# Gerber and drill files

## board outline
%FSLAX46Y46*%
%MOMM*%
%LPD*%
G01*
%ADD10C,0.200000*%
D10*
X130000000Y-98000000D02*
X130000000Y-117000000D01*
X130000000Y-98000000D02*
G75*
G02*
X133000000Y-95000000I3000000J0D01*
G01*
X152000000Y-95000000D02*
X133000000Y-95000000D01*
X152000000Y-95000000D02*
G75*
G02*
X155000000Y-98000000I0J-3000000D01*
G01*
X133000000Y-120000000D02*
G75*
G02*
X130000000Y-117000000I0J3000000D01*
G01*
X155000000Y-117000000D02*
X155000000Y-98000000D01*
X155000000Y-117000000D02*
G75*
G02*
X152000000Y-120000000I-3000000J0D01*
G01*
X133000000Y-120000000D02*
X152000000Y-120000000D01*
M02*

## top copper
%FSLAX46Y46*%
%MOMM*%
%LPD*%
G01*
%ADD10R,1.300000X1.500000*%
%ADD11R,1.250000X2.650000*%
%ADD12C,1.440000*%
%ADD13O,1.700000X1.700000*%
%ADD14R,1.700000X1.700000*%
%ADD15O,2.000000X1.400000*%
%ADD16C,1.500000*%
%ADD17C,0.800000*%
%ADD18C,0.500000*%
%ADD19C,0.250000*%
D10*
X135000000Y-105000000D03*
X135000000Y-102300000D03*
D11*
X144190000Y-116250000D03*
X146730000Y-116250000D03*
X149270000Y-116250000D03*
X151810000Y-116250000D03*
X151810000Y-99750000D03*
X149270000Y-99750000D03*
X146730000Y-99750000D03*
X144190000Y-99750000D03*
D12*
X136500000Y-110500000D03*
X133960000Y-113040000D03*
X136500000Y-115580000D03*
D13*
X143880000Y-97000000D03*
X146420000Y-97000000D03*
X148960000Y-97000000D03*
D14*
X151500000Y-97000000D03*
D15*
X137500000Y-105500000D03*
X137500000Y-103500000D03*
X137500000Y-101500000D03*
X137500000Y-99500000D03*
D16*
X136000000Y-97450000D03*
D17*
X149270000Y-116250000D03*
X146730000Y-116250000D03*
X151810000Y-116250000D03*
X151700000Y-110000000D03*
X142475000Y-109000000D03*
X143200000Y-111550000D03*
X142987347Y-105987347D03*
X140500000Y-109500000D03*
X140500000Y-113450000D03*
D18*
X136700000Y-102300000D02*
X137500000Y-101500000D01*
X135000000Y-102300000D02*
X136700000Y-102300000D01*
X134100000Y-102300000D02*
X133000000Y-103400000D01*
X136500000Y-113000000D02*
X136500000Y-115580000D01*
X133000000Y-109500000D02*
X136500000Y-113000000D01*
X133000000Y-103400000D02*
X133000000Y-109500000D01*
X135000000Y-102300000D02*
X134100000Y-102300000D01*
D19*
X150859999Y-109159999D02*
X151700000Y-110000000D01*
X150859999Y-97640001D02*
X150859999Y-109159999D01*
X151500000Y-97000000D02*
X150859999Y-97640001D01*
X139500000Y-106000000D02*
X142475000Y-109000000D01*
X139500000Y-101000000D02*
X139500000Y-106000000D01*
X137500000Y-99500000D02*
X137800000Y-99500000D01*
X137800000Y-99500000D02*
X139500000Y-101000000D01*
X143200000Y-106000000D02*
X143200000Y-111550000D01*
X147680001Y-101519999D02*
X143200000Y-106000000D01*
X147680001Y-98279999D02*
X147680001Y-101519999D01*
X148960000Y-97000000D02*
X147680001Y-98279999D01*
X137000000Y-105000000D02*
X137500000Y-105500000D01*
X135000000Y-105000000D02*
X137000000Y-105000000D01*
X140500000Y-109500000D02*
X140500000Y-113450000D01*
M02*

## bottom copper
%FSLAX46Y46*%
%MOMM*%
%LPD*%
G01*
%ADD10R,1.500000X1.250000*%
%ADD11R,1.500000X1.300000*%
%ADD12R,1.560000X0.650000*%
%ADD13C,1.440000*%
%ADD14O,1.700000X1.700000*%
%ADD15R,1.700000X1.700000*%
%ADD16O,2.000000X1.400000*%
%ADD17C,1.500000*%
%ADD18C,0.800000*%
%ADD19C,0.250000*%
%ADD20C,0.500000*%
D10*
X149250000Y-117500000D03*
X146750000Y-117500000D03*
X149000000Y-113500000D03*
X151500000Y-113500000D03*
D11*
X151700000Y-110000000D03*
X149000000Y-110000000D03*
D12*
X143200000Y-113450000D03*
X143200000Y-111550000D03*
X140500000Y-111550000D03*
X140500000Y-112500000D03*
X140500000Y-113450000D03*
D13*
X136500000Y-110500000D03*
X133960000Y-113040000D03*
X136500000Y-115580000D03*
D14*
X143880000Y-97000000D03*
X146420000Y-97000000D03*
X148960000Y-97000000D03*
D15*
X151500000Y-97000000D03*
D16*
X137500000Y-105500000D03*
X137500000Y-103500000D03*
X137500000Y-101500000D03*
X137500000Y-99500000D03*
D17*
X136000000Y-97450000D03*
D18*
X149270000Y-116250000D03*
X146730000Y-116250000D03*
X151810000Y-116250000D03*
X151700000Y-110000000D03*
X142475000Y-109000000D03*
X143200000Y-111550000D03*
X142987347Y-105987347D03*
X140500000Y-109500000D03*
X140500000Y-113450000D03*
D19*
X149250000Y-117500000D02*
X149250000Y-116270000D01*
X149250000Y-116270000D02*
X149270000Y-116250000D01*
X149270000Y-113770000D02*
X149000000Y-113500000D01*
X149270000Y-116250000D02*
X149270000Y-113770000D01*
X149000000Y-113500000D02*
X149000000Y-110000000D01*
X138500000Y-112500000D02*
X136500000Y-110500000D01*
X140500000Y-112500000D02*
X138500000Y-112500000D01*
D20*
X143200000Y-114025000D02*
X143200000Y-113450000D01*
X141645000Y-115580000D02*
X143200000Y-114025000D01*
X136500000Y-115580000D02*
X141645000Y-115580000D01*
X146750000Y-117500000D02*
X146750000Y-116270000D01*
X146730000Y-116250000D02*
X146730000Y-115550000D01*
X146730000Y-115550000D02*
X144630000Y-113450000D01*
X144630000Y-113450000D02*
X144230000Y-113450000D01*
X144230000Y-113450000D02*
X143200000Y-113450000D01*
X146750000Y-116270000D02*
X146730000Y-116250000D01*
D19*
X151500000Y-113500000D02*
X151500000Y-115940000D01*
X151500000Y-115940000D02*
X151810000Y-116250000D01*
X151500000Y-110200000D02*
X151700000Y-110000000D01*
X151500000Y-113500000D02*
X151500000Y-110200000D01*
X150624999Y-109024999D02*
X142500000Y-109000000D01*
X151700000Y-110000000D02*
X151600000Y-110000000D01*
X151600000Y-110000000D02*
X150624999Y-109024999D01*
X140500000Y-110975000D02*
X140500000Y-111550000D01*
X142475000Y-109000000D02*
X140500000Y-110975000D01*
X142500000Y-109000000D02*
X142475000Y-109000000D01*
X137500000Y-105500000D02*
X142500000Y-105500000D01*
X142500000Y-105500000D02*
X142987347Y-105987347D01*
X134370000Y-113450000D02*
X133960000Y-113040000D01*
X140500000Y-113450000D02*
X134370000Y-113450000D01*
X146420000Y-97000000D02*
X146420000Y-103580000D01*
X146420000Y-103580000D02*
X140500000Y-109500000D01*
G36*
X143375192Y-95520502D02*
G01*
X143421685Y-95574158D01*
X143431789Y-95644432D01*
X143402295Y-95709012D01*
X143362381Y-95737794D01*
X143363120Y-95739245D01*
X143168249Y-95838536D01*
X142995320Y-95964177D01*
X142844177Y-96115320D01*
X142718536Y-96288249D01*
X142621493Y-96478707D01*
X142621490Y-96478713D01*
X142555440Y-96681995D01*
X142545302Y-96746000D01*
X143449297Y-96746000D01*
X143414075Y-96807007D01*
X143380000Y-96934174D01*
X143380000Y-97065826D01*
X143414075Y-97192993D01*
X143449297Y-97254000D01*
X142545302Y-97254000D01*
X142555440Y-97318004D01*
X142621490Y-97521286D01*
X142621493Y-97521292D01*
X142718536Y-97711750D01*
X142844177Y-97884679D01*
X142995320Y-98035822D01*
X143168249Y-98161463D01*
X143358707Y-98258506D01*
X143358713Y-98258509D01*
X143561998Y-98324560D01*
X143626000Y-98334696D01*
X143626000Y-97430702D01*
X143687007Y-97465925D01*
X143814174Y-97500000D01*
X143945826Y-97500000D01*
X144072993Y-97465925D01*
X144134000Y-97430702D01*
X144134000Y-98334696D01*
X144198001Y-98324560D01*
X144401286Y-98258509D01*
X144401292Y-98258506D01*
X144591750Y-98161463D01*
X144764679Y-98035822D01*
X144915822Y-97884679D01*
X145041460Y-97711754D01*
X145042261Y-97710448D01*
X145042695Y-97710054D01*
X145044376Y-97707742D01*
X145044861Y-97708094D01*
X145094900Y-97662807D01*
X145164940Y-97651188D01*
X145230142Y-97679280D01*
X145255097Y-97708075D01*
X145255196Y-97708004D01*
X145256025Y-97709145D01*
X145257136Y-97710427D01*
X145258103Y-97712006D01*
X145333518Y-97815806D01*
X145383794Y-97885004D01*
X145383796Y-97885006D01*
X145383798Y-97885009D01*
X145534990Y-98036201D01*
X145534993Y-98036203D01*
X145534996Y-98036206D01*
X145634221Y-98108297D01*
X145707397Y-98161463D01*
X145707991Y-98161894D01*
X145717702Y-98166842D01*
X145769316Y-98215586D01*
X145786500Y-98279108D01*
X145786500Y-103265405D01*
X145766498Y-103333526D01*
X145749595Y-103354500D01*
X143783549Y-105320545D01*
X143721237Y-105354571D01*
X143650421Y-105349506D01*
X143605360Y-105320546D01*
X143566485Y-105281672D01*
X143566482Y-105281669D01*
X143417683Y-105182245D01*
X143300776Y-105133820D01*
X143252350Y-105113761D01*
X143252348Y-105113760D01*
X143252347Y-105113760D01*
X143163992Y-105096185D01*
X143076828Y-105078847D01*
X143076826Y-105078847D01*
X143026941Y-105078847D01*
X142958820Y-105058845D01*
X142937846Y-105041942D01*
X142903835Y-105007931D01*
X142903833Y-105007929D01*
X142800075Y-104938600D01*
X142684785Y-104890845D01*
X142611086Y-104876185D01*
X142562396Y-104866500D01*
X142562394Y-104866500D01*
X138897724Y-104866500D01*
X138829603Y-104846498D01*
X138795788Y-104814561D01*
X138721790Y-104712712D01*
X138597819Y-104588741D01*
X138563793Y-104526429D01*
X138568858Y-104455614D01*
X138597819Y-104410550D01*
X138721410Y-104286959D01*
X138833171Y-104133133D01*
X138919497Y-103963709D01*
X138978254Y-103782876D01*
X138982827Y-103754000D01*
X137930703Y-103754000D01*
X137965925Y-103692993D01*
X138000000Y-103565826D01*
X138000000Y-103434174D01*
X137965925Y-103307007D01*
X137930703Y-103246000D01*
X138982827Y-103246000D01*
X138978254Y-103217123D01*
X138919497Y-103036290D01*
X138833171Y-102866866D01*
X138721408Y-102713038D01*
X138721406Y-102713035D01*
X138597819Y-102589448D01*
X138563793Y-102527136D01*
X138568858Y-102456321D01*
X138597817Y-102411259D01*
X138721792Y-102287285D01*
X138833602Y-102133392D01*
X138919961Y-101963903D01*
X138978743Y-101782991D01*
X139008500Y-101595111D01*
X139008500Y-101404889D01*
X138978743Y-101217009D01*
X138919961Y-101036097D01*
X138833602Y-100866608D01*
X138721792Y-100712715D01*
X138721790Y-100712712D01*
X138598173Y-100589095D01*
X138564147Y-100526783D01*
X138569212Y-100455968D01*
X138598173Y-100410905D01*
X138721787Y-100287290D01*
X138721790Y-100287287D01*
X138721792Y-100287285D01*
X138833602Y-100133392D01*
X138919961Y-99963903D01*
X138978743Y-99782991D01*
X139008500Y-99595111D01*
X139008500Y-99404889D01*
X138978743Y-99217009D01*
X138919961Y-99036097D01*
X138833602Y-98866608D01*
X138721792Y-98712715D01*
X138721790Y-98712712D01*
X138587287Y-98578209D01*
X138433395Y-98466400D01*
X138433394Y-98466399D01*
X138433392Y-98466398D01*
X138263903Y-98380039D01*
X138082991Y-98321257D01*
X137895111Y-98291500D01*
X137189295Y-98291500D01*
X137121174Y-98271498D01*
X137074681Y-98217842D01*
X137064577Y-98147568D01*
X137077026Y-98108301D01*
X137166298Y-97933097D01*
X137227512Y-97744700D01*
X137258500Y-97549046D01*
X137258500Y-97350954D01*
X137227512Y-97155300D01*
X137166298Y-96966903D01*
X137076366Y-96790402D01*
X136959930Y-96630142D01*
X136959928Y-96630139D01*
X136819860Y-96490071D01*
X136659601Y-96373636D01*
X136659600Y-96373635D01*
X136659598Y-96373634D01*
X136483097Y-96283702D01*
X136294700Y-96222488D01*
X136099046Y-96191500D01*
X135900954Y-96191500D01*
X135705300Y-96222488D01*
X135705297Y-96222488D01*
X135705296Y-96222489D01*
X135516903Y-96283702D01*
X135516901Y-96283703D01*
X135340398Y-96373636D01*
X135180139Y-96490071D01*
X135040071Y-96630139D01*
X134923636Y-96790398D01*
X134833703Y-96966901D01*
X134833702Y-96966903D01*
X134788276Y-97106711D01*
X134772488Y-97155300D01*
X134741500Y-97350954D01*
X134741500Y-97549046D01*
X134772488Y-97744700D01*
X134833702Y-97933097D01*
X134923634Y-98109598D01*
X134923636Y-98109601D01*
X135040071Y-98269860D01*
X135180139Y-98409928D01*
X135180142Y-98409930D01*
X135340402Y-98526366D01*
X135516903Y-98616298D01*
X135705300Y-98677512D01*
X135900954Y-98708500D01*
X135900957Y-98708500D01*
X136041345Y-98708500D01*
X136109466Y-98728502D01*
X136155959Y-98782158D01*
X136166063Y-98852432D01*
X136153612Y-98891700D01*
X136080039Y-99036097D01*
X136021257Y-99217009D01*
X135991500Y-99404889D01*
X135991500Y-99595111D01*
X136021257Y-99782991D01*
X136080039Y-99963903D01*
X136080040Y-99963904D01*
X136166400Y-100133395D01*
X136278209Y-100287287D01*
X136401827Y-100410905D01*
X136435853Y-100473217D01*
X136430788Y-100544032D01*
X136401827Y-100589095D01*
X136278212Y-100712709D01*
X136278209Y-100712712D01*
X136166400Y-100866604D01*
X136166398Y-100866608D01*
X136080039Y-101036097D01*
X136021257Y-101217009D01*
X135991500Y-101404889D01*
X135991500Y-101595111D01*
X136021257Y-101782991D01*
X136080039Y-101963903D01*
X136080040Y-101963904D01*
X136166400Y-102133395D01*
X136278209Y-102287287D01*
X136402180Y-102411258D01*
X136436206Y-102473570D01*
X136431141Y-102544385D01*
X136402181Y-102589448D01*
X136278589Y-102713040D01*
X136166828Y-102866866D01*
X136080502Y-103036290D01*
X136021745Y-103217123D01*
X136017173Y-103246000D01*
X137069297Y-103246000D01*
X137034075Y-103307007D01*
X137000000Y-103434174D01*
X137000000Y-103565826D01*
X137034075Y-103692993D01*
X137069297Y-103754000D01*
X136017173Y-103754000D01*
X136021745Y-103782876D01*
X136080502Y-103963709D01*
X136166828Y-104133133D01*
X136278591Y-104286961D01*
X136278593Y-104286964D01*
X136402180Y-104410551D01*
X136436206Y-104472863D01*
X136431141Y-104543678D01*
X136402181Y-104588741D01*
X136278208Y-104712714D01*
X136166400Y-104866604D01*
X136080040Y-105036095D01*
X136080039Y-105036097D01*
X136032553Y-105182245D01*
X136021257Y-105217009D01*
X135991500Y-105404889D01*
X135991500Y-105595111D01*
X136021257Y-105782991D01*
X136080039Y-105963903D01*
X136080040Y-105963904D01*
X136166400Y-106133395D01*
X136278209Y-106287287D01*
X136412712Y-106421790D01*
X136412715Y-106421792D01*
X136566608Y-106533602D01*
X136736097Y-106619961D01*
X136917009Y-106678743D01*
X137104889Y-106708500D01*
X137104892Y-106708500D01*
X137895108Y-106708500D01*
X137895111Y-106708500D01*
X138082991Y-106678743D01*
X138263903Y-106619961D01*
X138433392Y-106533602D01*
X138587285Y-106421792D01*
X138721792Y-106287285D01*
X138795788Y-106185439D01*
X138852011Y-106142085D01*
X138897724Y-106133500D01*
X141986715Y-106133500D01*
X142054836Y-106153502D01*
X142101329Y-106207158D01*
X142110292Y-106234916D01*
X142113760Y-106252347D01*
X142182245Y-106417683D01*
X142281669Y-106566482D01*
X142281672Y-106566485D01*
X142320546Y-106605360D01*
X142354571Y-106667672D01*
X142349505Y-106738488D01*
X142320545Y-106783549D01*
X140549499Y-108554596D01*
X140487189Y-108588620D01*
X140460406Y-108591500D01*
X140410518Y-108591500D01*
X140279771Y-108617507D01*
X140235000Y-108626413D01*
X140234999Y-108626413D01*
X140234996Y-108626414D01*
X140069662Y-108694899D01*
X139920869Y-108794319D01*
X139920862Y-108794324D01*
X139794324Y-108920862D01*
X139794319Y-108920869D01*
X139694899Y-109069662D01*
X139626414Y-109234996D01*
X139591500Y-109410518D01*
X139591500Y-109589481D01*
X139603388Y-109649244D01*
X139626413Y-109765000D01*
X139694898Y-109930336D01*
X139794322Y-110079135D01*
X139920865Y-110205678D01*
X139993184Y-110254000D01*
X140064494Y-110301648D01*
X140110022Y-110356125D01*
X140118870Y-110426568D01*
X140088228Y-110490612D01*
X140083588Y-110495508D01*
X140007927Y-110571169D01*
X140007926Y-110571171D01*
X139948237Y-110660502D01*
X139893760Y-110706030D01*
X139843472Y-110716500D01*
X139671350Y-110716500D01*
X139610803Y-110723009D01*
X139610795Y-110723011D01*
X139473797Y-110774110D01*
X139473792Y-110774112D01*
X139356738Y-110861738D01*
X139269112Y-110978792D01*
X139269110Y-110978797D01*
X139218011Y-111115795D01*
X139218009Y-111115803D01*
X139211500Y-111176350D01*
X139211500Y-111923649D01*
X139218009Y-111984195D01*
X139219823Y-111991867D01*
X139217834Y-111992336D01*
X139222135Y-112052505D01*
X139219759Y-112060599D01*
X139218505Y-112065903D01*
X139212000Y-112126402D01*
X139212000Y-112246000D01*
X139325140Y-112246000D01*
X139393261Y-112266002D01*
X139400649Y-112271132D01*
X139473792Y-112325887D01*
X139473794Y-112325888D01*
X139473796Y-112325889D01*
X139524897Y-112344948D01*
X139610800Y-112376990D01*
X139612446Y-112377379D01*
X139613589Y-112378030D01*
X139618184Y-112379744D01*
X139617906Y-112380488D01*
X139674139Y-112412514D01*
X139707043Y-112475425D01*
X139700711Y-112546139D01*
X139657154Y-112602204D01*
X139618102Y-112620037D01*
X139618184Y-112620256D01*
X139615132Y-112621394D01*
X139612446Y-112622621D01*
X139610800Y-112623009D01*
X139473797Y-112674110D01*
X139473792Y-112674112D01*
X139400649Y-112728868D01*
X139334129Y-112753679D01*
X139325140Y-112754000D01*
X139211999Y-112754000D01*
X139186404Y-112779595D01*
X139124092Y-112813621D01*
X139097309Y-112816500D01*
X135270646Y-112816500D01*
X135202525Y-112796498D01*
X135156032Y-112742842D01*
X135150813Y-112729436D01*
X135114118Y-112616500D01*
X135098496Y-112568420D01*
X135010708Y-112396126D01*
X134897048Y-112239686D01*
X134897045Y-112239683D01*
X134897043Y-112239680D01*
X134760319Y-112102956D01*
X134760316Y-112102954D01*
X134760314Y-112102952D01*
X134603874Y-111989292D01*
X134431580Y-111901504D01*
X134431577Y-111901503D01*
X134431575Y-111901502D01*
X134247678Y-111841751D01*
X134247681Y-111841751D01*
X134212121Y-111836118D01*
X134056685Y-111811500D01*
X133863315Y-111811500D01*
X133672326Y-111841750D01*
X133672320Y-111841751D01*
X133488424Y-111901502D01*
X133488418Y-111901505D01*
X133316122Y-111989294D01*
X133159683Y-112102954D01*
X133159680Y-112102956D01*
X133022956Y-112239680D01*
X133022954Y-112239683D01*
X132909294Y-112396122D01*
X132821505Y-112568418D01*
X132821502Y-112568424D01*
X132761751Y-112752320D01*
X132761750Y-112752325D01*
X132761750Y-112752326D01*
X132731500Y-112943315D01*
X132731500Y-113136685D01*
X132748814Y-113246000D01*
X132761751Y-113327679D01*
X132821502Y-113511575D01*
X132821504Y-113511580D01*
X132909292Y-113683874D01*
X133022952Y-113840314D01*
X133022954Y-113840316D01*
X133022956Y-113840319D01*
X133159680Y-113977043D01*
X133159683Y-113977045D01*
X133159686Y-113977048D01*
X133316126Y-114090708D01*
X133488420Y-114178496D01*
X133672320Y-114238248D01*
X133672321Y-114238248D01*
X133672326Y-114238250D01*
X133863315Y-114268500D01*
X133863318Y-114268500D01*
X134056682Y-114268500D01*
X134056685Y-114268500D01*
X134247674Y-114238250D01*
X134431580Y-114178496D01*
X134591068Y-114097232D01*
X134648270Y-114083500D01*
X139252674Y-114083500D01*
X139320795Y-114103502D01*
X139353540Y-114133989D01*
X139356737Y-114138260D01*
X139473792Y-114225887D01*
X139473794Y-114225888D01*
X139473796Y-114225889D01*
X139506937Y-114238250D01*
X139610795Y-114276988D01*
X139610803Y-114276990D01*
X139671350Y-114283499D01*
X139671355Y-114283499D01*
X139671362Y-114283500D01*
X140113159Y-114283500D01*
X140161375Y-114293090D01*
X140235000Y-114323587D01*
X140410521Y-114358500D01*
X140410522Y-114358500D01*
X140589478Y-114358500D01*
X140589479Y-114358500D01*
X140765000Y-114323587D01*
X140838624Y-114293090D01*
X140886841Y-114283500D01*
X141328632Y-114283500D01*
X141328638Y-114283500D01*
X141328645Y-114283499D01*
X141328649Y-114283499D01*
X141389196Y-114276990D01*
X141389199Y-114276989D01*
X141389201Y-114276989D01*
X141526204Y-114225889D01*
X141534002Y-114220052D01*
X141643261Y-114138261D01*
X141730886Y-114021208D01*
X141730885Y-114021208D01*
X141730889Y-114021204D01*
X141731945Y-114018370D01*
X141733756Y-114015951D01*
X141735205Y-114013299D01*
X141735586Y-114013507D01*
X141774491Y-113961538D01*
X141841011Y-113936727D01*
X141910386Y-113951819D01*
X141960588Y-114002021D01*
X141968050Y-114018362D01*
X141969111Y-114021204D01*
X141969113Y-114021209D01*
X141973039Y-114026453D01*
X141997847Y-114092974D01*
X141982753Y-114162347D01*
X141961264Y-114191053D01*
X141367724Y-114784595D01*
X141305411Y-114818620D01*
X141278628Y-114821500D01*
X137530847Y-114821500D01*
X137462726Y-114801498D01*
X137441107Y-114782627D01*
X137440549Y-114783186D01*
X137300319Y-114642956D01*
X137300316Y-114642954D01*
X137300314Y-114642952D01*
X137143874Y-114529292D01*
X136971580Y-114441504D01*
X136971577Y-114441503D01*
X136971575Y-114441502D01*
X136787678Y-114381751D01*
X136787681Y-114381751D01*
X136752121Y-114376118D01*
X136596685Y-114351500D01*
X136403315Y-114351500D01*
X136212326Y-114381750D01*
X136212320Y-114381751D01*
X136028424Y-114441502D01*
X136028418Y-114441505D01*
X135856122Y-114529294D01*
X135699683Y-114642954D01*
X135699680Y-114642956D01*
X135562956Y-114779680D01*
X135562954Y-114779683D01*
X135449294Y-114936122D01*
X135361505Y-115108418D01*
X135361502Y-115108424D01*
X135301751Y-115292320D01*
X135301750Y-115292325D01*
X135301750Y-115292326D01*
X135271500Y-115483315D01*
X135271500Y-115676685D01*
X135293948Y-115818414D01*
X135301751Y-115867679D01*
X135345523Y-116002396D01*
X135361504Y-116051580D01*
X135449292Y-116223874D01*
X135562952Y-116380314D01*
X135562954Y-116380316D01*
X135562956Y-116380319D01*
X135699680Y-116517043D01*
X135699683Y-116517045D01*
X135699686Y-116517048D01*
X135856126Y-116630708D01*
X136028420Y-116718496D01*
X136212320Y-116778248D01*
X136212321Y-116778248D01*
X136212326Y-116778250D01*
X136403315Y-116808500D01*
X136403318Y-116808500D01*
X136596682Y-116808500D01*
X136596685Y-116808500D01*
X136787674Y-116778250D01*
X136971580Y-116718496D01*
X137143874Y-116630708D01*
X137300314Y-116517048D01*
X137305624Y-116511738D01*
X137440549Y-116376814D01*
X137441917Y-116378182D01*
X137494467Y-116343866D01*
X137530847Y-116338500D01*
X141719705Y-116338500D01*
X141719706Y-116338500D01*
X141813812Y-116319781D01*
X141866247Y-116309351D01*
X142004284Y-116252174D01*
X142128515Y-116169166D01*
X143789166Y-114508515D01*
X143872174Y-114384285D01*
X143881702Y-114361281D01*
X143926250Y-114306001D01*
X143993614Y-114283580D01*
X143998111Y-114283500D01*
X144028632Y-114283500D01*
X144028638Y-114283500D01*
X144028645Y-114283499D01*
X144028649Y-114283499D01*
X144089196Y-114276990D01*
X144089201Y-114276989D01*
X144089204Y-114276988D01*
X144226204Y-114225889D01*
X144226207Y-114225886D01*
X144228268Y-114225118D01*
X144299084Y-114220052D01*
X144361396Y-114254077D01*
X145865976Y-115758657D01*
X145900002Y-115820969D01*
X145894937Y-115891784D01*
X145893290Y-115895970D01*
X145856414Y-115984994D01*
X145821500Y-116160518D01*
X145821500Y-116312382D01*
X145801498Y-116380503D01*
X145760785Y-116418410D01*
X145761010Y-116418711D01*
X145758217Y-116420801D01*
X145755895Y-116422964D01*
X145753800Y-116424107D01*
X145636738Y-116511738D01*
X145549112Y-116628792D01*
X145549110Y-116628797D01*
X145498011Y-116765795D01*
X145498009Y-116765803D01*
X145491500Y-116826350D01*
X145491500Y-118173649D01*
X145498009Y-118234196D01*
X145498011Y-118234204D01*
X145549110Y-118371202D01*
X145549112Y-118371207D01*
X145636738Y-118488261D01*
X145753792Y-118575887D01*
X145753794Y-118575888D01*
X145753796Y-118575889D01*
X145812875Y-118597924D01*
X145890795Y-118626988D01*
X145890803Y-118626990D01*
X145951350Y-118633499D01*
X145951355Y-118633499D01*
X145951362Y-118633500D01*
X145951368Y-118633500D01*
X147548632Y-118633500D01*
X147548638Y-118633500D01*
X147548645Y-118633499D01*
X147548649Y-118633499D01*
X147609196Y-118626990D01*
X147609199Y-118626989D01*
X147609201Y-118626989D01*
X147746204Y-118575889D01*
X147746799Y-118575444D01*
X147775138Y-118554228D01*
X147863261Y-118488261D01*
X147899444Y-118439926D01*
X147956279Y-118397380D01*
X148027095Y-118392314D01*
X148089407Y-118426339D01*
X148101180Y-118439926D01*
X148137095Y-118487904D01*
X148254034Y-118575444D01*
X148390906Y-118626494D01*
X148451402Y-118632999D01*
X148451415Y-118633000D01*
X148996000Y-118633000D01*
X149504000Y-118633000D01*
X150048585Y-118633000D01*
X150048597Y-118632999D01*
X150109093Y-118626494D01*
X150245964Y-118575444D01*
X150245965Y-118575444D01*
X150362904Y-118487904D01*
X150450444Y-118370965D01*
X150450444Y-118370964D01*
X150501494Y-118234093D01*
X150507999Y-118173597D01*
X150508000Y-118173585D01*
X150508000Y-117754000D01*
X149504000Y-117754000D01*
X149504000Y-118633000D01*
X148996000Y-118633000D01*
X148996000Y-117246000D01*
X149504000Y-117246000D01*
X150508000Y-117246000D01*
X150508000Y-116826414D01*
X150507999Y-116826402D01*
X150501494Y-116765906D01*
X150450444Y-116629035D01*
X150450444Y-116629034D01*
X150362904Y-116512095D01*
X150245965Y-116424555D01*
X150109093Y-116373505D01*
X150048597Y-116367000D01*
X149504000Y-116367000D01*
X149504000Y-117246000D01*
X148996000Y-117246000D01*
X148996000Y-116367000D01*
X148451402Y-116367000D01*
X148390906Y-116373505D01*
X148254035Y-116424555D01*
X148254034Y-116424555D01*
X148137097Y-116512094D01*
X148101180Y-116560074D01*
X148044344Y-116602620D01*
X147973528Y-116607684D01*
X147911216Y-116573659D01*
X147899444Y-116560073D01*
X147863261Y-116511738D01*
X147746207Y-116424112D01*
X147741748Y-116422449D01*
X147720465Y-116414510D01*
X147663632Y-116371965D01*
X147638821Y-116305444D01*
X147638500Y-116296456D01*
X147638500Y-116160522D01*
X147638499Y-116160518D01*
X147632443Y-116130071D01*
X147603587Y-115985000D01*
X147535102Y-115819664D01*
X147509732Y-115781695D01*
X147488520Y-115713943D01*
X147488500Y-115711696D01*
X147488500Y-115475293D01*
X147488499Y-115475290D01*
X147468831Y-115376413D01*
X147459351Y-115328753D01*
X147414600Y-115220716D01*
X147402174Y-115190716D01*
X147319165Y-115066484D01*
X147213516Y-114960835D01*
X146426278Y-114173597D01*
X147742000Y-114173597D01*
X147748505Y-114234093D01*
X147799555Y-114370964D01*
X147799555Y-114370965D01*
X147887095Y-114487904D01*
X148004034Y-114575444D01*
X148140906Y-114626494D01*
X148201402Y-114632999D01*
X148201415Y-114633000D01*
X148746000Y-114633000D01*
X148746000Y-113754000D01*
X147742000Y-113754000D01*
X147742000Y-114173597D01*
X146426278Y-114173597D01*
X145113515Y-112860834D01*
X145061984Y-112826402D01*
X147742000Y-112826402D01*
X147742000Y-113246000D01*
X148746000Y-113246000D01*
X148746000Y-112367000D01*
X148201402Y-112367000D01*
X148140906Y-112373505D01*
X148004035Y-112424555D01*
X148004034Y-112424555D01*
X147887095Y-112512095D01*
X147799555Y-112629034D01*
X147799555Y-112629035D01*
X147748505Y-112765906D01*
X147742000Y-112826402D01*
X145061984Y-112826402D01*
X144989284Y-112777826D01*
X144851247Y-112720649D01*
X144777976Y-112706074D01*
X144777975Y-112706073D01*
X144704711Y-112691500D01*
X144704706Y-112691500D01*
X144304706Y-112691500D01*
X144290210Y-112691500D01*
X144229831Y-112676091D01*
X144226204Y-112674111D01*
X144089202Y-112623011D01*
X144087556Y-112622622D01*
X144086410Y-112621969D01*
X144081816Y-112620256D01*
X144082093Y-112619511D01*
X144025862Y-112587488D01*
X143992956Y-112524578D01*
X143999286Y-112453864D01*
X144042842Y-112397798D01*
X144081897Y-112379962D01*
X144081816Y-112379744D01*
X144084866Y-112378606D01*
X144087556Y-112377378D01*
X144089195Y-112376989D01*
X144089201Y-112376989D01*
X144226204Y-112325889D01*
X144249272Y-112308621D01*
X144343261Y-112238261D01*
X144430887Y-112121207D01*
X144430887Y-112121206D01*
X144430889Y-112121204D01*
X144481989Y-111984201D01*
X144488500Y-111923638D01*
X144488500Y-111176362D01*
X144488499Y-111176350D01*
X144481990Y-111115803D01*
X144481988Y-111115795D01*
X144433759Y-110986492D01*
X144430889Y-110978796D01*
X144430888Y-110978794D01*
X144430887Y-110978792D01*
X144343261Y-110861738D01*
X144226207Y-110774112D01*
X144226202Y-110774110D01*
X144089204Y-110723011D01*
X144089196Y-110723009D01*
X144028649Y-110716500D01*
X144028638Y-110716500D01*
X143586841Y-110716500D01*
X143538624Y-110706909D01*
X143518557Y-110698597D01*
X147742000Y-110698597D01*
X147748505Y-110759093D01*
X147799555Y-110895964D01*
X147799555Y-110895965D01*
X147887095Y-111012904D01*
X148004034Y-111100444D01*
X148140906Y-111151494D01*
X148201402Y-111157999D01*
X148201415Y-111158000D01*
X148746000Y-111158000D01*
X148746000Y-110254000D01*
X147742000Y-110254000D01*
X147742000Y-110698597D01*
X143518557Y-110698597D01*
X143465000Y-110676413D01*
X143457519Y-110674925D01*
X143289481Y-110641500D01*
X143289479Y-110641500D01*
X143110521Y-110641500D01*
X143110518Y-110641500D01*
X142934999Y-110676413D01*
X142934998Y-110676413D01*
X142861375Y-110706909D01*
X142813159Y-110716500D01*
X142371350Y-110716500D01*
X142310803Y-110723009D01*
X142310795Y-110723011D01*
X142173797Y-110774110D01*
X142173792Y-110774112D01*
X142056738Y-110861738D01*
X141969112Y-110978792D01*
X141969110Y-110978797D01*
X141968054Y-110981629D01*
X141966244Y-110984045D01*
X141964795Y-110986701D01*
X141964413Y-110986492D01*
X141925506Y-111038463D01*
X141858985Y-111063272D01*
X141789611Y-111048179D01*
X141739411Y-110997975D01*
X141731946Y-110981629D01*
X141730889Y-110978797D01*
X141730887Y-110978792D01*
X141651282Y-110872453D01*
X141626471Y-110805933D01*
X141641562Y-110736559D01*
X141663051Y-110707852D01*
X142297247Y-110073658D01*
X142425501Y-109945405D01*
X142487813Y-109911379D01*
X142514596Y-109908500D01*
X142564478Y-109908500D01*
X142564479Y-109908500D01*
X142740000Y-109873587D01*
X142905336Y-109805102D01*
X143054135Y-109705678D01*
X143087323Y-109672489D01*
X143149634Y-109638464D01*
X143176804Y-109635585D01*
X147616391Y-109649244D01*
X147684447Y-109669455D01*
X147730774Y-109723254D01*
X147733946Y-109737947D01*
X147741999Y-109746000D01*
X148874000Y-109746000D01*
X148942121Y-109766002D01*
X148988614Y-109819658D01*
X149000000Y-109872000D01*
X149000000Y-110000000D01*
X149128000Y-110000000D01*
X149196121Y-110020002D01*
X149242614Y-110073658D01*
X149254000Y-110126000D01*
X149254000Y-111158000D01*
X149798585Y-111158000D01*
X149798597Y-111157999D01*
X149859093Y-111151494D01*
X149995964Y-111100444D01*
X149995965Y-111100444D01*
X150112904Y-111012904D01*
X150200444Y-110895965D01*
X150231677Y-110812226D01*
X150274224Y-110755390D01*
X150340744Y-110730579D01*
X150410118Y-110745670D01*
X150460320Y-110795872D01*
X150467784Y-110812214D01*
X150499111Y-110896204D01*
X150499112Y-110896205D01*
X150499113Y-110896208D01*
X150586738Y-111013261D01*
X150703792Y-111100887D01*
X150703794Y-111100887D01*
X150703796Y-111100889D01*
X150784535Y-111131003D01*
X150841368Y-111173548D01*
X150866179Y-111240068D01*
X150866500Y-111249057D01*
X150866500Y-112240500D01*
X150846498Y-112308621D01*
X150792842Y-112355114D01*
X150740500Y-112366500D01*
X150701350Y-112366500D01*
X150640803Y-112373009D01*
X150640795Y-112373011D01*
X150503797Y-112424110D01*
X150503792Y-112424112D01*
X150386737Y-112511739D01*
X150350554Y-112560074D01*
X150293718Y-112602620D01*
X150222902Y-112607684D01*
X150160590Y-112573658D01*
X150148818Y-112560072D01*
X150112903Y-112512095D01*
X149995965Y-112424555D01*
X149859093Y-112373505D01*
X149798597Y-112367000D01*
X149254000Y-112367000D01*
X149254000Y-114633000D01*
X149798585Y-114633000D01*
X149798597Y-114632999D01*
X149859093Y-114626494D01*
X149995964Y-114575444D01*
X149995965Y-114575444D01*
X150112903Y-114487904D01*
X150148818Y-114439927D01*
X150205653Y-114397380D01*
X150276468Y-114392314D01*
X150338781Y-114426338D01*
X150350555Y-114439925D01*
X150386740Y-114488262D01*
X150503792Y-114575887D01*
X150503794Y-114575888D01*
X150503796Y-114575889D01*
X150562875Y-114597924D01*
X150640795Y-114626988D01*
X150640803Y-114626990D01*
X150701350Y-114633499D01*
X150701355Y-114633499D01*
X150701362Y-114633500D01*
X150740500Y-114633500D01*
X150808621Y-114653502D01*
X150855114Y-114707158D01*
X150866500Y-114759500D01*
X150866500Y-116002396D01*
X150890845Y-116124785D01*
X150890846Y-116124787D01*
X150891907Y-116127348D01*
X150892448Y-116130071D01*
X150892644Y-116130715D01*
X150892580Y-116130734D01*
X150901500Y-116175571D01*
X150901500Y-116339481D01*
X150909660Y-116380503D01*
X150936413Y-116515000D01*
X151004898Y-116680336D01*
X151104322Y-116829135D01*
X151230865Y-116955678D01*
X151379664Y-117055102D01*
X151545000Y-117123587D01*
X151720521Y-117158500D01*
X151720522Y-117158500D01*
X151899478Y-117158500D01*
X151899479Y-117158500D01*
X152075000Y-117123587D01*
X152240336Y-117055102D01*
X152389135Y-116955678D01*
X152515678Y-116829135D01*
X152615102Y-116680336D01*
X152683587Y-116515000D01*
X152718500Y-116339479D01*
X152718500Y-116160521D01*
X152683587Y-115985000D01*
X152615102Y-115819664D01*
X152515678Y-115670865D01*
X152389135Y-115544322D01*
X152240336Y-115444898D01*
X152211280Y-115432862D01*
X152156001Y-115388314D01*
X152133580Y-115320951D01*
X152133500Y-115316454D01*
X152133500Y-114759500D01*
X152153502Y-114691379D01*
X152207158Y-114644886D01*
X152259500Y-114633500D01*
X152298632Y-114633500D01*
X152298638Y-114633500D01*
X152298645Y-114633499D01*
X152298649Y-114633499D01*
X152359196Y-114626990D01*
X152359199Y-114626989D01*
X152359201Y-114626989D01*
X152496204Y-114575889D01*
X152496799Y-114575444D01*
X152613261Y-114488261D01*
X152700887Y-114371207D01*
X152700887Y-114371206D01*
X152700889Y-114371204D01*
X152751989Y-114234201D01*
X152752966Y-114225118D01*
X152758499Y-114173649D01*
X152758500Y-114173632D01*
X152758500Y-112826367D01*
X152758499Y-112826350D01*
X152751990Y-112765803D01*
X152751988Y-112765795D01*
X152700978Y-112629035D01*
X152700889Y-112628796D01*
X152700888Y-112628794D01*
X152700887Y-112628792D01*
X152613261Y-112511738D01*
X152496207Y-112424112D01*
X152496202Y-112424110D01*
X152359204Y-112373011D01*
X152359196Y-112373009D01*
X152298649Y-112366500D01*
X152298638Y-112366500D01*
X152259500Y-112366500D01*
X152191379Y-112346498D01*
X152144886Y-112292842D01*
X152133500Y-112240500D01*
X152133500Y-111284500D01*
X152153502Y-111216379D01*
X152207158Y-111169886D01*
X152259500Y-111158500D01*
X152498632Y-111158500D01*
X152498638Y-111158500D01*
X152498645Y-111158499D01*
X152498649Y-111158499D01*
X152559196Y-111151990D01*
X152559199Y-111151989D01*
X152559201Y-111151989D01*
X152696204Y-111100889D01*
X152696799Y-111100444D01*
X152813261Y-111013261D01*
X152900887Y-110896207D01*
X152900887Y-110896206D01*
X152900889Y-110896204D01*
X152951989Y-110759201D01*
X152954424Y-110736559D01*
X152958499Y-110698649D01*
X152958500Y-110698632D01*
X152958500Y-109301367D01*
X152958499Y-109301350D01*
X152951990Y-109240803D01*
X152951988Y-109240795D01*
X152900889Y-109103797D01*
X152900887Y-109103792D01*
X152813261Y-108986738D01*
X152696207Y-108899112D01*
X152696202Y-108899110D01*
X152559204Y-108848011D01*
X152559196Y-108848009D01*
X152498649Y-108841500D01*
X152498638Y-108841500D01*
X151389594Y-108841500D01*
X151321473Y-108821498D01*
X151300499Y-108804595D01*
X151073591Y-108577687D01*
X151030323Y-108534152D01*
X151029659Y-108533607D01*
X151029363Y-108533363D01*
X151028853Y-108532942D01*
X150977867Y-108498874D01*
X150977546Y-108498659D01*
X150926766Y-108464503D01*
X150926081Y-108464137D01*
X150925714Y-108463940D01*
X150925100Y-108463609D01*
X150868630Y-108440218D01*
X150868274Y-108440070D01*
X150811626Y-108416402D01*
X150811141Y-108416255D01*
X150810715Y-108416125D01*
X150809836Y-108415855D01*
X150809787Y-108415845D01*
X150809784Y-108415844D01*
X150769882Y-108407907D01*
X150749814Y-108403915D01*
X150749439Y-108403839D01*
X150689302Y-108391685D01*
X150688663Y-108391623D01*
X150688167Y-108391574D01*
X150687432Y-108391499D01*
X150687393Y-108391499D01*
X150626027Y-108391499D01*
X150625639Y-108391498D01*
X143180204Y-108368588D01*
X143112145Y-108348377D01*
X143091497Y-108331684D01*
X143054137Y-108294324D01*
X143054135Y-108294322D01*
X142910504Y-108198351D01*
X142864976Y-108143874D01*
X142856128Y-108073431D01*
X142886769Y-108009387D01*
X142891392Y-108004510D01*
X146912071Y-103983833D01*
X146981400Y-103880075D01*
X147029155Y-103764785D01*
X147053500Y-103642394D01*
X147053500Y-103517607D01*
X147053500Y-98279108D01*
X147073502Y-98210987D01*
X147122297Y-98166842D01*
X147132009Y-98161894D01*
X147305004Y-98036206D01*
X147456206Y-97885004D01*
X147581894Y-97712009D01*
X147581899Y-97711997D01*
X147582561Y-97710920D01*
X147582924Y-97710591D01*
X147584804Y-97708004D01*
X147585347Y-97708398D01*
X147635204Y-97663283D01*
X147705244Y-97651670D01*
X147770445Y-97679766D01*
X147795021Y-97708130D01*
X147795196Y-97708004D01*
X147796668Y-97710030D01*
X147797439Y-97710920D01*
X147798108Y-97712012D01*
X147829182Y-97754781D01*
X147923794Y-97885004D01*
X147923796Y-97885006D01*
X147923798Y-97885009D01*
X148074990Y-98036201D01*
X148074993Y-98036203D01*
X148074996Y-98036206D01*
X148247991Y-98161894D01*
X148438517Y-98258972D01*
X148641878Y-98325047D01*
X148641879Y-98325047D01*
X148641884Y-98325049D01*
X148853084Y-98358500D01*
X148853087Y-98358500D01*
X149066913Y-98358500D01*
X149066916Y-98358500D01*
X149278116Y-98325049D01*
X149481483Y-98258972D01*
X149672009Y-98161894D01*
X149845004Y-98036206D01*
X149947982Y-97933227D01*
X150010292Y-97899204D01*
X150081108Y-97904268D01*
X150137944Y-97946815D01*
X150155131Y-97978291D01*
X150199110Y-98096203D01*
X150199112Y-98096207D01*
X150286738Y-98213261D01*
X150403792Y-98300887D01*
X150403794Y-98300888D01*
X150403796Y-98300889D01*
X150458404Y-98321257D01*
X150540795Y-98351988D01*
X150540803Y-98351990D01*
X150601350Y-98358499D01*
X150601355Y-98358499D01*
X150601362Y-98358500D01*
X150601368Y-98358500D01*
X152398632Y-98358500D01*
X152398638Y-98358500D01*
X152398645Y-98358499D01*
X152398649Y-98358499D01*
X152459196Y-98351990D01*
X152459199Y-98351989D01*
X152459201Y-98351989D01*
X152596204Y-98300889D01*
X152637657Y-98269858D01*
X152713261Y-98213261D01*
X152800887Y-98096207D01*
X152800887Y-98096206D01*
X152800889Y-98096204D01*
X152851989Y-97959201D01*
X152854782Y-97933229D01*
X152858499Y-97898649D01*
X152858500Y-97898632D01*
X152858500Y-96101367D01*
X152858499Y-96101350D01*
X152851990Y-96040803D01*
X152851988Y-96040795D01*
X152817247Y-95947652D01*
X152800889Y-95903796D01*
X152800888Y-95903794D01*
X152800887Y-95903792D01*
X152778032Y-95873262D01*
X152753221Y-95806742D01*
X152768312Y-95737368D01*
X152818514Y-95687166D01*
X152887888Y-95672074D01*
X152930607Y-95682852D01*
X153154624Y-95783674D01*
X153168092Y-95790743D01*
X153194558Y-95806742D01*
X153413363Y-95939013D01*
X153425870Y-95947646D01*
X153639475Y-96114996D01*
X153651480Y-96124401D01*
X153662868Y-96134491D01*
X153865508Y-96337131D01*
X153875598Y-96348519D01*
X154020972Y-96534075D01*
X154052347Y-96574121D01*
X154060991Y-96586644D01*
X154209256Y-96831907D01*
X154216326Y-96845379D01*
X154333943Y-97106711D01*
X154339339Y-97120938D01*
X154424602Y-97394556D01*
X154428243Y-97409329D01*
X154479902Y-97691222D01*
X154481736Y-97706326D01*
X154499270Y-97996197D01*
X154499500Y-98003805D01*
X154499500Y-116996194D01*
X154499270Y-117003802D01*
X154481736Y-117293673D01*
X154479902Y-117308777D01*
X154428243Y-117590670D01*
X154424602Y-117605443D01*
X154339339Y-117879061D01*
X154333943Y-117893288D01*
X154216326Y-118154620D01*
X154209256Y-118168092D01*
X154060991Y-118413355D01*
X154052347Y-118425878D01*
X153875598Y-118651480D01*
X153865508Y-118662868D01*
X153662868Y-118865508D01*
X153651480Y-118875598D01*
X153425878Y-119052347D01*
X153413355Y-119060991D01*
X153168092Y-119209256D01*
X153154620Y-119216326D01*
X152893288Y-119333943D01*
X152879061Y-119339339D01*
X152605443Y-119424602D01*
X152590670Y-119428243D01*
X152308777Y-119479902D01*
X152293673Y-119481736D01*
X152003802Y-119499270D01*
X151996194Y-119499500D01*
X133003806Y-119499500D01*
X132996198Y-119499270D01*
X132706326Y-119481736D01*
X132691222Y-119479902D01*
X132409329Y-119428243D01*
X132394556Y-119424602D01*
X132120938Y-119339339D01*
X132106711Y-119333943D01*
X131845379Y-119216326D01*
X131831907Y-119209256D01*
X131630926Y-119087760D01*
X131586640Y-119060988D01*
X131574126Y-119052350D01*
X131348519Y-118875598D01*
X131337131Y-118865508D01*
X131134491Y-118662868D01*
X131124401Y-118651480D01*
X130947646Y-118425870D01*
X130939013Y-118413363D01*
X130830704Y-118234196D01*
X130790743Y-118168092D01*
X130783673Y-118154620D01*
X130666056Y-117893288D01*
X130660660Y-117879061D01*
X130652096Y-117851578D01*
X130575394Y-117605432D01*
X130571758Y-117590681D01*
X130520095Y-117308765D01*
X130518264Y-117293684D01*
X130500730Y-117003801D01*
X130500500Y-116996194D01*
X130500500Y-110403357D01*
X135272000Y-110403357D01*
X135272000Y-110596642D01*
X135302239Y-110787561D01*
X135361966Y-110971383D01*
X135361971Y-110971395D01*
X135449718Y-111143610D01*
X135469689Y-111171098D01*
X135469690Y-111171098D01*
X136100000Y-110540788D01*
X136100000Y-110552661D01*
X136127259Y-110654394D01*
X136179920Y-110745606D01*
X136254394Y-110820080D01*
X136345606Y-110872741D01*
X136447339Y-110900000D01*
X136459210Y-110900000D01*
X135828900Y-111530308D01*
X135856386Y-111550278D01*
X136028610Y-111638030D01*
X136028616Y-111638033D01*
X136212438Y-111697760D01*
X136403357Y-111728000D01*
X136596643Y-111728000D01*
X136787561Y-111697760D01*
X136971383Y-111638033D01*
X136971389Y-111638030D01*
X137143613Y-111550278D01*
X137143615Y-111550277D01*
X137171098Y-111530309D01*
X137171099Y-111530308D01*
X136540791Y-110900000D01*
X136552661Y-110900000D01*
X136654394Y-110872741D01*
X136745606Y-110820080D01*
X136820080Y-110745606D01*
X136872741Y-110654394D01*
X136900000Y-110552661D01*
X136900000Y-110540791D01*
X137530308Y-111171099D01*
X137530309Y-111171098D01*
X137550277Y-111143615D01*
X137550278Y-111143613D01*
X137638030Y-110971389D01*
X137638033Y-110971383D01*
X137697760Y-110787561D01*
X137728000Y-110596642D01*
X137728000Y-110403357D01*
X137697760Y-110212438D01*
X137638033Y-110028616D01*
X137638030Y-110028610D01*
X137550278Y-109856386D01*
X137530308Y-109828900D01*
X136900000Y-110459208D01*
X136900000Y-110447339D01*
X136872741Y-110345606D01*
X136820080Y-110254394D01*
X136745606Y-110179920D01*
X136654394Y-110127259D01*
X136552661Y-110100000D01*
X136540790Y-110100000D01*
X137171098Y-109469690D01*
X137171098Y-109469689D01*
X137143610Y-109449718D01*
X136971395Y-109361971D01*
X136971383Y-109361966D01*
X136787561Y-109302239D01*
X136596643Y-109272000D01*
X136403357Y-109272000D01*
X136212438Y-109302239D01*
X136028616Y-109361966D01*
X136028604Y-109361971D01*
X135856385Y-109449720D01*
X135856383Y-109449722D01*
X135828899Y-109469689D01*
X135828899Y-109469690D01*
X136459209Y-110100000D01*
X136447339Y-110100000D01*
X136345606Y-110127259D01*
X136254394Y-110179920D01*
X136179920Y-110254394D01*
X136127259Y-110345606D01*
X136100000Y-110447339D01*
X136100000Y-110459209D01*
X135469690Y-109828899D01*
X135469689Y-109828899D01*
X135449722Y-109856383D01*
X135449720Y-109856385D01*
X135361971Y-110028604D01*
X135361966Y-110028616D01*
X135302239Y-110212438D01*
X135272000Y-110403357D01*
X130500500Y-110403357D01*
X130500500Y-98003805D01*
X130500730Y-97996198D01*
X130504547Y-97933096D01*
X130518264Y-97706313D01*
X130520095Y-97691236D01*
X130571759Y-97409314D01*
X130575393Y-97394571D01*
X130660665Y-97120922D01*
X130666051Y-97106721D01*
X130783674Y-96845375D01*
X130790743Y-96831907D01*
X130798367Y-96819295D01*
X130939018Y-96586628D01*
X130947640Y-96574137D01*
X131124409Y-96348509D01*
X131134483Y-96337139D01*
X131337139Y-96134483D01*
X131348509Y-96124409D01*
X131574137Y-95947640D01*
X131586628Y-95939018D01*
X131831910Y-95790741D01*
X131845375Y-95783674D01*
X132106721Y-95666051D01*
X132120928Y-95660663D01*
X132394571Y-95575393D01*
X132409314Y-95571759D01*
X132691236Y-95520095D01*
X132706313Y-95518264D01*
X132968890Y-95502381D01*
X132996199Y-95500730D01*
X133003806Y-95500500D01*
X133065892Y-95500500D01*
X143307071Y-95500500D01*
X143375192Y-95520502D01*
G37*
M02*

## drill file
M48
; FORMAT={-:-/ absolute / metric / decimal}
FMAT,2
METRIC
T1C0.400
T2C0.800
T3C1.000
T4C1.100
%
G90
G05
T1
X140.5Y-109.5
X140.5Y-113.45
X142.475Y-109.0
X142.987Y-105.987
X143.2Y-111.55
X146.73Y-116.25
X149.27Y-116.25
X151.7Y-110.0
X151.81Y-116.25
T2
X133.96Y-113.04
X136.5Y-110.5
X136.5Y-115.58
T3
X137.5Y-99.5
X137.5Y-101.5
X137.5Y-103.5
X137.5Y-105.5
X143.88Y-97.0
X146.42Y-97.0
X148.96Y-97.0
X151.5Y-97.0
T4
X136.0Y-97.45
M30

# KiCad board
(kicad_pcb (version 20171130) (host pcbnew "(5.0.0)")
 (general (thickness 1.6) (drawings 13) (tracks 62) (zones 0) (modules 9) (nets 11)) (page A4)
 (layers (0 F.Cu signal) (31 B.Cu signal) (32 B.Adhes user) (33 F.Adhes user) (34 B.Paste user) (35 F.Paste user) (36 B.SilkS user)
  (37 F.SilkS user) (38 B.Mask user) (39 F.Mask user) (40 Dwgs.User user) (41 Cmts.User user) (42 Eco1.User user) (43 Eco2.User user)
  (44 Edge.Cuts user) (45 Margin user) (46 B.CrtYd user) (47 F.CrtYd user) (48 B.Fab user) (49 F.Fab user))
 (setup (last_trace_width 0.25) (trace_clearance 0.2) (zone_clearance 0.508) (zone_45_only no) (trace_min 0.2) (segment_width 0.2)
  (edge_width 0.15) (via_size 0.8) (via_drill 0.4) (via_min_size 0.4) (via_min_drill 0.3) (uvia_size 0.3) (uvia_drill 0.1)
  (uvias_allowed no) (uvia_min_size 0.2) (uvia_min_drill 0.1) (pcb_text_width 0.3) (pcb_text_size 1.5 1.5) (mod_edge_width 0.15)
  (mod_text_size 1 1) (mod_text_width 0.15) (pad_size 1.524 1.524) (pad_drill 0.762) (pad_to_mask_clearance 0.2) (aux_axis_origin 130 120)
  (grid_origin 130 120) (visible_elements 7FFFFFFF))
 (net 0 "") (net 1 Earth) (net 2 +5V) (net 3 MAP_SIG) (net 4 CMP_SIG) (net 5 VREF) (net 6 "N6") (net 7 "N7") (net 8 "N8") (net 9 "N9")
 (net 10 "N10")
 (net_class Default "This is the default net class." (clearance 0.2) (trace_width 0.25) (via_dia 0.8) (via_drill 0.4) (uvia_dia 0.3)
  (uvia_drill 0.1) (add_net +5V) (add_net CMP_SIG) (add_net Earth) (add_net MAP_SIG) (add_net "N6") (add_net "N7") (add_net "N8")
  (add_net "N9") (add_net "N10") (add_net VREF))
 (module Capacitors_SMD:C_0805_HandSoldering (layer B.Cu) (at 148 117.5)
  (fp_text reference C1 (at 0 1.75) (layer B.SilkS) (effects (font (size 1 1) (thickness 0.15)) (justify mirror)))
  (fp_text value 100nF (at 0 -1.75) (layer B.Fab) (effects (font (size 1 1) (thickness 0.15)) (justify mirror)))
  (pad 2 smd rect (at 1.25 0) (size 1.5 1.25) (layers B.Cu B.Paste B.Mask) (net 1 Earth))
  (pad 1 smd rect (at -1.25 0) (size 1.5 1.25) (layers B.Cu B.Paste B.Mask) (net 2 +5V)))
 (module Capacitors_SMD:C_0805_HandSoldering (layer B.Cu) (at 150.25 113.5)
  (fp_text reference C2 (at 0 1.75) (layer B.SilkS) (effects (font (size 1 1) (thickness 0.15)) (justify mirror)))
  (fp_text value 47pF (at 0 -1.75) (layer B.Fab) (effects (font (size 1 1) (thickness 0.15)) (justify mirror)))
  (pad 1 smd rect (at -1.25 0) (size 1.5 1.25) (layers B.Cu B.Paste B.Mask) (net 1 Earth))
  (pad 2 smd rect (at 1.25 0) (size 1.5 1.25) (layers B.Cu B.Paste B.Mask) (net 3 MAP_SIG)))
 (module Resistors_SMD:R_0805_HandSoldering (layer F.Cu) (at 135 103.65 270)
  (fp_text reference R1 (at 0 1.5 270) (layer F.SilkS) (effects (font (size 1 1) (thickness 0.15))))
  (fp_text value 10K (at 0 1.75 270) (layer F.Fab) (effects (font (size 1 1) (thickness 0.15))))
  (pad 2 smd rect (at 1.35 0 270) (size 1.5 1.3) (layers F.Cu F.Paste F.Mask) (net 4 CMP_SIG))
  (pad 1 smd rect (at -1.35 0 270) (size 1.5 1.3) (layers F.Cu F.Paste F.Mask) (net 2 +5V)))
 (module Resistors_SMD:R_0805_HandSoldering (layer B.Cu) (at 150.35 110 180)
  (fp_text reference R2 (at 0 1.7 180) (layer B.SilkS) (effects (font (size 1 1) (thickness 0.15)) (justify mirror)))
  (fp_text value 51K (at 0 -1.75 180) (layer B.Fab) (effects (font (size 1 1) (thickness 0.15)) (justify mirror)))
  (pad 1 smd rect (at -1.35 0 180) (size 1.5 1.3) (layers B.Cu B.Paste B.Mask) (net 3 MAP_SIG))
  (pad 2 smd rect (at 1.35 0 180) (size 1.5 1.3) (layers B.Cu B.Paste B.Mask) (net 1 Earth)))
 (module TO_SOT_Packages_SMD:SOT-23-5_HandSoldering (layer B.Cu) (at 141.85 112.5)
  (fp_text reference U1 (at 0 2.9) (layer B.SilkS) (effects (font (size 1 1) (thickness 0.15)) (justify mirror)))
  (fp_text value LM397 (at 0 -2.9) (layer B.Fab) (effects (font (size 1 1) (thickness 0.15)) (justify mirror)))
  (pad 5 smd rect (at 1.35 0.95) (size 1.56 0.65) (layers B.Cu B.Paste B.Mask) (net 2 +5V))
  (pad 4 smd rect (at 1.35 -0.95) (size 1.56 0.65) (layers B.Cu B.Paste B.Mask) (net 4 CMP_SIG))
  (pad 3 smd rect (at -1.35 -0.95) (size 1.56 0.65) (layers B.Cu B.Paste B.Mask) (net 3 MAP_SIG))
  (pad 2 smd rect (at -1.35 0) (size 1.56 0.65) (layers B.Cu B.Paste B.Mask) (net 1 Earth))
  (pad 1 smd rect (at -1.35 0.95) (size 1.56 0.65) (layers B.Cu B.Paste B.Mask) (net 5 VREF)))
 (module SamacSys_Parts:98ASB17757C (layer F.Cu) (at 148 108 90)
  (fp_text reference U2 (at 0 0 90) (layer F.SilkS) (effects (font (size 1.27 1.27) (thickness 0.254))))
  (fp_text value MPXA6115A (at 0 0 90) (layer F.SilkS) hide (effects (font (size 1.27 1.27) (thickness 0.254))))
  (pad 1 smd rect (at -8.25 -3.81 180) (size 1.25 2.65) (layers F.Cu F.Paste F.Mask) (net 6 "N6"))
  (pad 2 smd rect (at -8.25 -1.27 180) (size 1.25 2.65) (layers F.Cu F.Paste F.Mask) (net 2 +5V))
  (pad 3 smd rect (at -8.25 1.27 180) (size 1.25 2.65) (layers F.Cu F.Paste F.Mask) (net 1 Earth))
  (pad 4 smd rect (at -8.25 3.81 180) (size 1.25 2.65) (layers F.Cu F.Paste F.Mask) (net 3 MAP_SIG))
  (pad 5 smd rect (at 8.25 3.81 180) (size 1.25 2.65) (layers F.Cu F.Paste F.Mask) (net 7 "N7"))
  (pad 6 smd rect (at 8.25 1.27 180) (size 1.25 2.65) (layers F.Cu F.Paste F.Mask) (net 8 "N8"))
  (pad 7 smd rect (at 8.25 -1.27 180) (size 1.25 2.65) (layers F.Cu F.Paste F.Mask) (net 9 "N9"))
  (pad 8 smd rect (at 8.25 -3.81 180) (size 1.25 2.65) (layers F.Cu F.Paste F.Mask) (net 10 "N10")))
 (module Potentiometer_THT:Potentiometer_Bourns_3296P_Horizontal (layer F.Cu) (at 136.5 110.5)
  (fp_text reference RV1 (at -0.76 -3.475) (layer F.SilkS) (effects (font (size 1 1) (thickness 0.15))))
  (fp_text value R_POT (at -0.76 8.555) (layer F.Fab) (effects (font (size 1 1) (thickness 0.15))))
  (pad 1 thru_hole circle (at 0 0) (size 1.44 1.44) (drill 0.8) (layers *.Cu *.Mask) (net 1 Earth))
  (pad 2 thru_hole circle (at -2.54 2.54) (size 1.44 1.44) (drill 0.8) (layers *.Cu *.Mask) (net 5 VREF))
  (pad 3 thru_hole circle (at 0 5.08) (size 1.44 1.44) (drill 0.8) (layers *.Cu *.Mask) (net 2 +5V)))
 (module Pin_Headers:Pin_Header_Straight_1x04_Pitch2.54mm (layer F.Cu) (at 151.5 97 270)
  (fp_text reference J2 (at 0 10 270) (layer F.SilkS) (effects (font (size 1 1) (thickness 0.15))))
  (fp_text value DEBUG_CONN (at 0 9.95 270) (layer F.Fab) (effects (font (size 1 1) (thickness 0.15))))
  (pad 4 thru_hole oval (at 0 7.62 270) (size 1.7 1.7) (drill 1) (layers *.Cu *.Mask) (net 1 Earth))
  (pad 3 thru_hole oval (at 0 5.08 270) (size 1.7 1.7) (drill 1) (layers *.Cu *.Mask) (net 5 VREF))
  (pad 2 thru_hole oval (at 0 2.54 270) (size 1.7 1.7) (drill 1) (layers *.Cu *.Mask) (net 4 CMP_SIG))
  (pad 1 thru_hole rect (at 0 0 270) (size 1.7 1.7) (drill 1) (layers *.Cu *.Mask) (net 3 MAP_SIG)))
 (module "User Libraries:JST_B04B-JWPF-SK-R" (layer B.Cu) (at 137.5 102.5 90)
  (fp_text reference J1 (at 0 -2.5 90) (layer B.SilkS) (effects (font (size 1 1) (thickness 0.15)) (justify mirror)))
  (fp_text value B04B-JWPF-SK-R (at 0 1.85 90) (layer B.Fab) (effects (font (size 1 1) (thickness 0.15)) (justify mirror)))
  (pad 1 thru_hole oval (at -3 0 90) (size 1.4 2) (drill 1) (layers *.Cu *.Mask) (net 4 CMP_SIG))
  (pad 2 thru_hole oval (at -1 0 90) (size 1.4 2) (drill 1) (layers *.Cu *.Mask) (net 1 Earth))
  (pad 3 thru_hole oval (at 1 0 90) (size 1.4 2) (drill 1) (layers *.Cu *.Mask) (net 2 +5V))
  (pad 4 thru_hole oval (at 3 0 90) (size 1.4 2) (drill 1) (layers *.Cu *.Mask) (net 3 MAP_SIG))
  (pad "" thru_hole circle (at 5.05 -1.5 90) (size 1.5 1.5) (drill 1.1) (layers *.Cu *.Mask)))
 (gr_line (start 130 98) (end 130 117) (layer Edge.Cuts) (width 0.2))
 (gr_arc (start 133 98) (end 133 95) (angle -90.000002) (layer Edge.Cuts) (width 0.2))
 (gr_line (start 152 95) (end 133 95) (layer Edge.Cuts) (width 0.2))
 (gr_arc (start 152 98) (end 155 98) (angle -90.000003) (layer Edge.Cuts) (width 0.2))
 (gr_arc (start 133 117) (end 130 117) (angle -89.999992) (layer Edge.Cuts) (width 0.2))
 (gr_line (start 155 117) (end 155 98) (layer Edge.Cuts) (width 0.2))
 (gr_arc (start 152 117) (end 152 120) (angle -90.000003) (layer Edge.Cuts) (width 0.2))
 (gr_line (start 133 120) (end 152 120) (layer Edge.Cuts) (width 0.2))
 (via (at 149.27 116.25) (size 0.8) (drill 0.4) (layers F.Cu B.Cu) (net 1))
 (segment (start 149.25 117.5) (end 149.25 116.27) (width 0.25) (layer B.Cu) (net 1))
 (segment (start 149.25 116.27) (end 149.27 116.25) (width 0.25) (layer B.Cu) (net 1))
 (segment (start 149.27 113.77) (end 149 113.5) (width 0.25) (layer B.Cu) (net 1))
 (segment (start 149.27 116.25) (end 149.27 113.77) (width 0.25) (layer B.Cu) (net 1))
 (segment (start 149 113.5) (end 149 110) (width 0.25) (layer B.Cu) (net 1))
 (segment (start 138.5 112.5) (end 136.5 110.5) (width 0.25) (layer B.Cu) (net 1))
 (segment (start 140.5 112.5) (end 138.5 112.5) (width 0.25) (layer B.Cu) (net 1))
 (segment (start 143.2 114.025) (end 143.2 113.45) (width 0.5) (layer B.Cu) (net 2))
 (segment (start 141.645 115.58) (end 143.2 114.025) (width 0.5) (layer B.Cu) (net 2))
 (segment (start 136.5 115.58) (end 141.645 115.58) (width 0.5) (layer B.Cu) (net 2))
 (segment (start 146.75 117.5) (end 146.75 116.27) (width 0.5) (layer B.Cu) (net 2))
 (via (at 146.73 116.25) (size 0.8) (drill 0.4) (layers F.Cu B.Cu) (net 2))
 (segment (start 146.73 116.25) (end 146.73 115.55) (width 0.5) (layer B.Cu) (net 2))
 (segment (start 146.73 115.55) (end 144.63 113.45) (width 0.5) (layer B.Cu) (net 2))
 (segment (start 144.63 113.45) (end 144.23 113.45) (width 0.5) (layer B.Cu) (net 2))
 (segment (start 144.23 113.45) (end 143.2 113.45) (width 0.5) (layer B.Cu) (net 2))
 (segment (start 146.75 116.27) (end 146.73 116.25) (width 0.5) (layer B.Cu) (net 2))
 (segment (start 136.7 102.3) (end 137.5 101.5) (width 0.5) (layer F.Cu) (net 2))
 (segment (start 135 102.3) (end 136.7 102.3) (width 0.5) (layer F.Cu) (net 2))
 (segment (start 134.1 102.3) (end 133 103.4) (width 0.5) (layer F.Cu) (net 2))
 (segment (start 136.5 113) (end 136.5 115.58) (width 0.5) (layer F.Cu) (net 2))
 (segment (start 133 109.5) (end 136.5 113) (width 0.5) (layer F.Cu) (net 2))
 (segment (start 133 103.4) (end 133 109.5) (width 0.5) (layer F.Cu) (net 2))
 (segment (start 135 102.3) (end 134.1 102.3) (width 0.5) (layer F.Cu) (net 2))
 (via (at 151.81 116.25) (size 0.8) (drill 0.4) (layers F.Cu B.Cu) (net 3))
 (segment (start 151.5 113.5) (end 151.5 115.94) (width 0.25) (layer B.Cu) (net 3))
 (segment (start 151.5 115.94) (end 151.81 116.25) (width 0.25) (layer B.Cu) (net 3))
 (segment (start 151.5 110.2) (end 151.7 110) (width 0.25) (layer B.Cu) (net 3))
 (segment (start 151.5 113.5) (end 151.5 110.2) (width 0.25) (layer B.Cu) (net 3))
 (via (at 151.7 110) (size 0.8) (drill 0.4) (layers F.Cu B.Cu) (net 3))
 (segment (start 150.859999 109.159999) (end 151.7 110) (width 0.25) (layer F.Cu) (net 3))
 (segment (start 150.859999 97.640001) (end 150.859999 109.159999) (width 0.25) (layer F.Cu) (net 3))
 (segment (start 151.5 97) (end 150.859999 97.640001) (width 0.25) (layer F.Cu) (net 3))
 (segment (start 150.624999 109.024999) (end 142.5 109) (width 0.25) (layer B.Cu) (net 3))
 (segment (start 151.7 110) (end 151.6 110) (width 0.25) (layer B.Cu) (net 3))
 (segment (start 151.6 110) (end 150.624999 109.024999) (width 0.25) (layer B.Cu) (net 3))
 (segment (start 140.5 110.975) (end 140.5 111.55) (width 0.25) (layer B.Cu) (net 3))
 (segment (start 142.475 109) (end 140.5 110.975) (width 0.25) (layer B.Cu) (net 3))
 (segment (start 142.5 109) (end 142.475 109) (width 0.25) (layer B.Cu) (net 3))
 (via (at 142.475 109) (size 0.8) (drill 0.4) (layers F.Cu B.Cu) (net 3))
 (segment (start 139.5 106) (end 142.475 109) (width 0.25) (layer F.Cu) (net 3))
 (segment (start 139.5 101) (end 139.5 106) (width 0.25) (layer F.Cu) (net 3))
 (segment (start 137.5 99.5) (end 137.8 99.5) (width 0.25) (layer F.Cu) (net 3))
 (segment (start 137.8 99.5) (end 139.5 101) (width 0.25) (layer F.Cu) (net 3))
 (via (at 143.2 111.55) (size 0.8) (drill 0.4) (layers F.Cu B.Cu) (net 4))
 (segment (start 143.2 106) (end 143.2 111.55) (width 0.25) (layer F.Cu) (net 4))
 (segment (start 147.680001 101.519999) (end 143.2 106) (width 0.25) (layer F.Cu) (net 4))
 (segment (start 147.680001 98.279999) (end 147.680001 101.519999) (width 0.25) (layer F.Cu) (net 4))
 (segment (start 148.96 97) (end 147.680001 98.279999) (width 0.25) (layer F.Cu) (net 4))
 (via (at 142.987347 105.987347) (size 0.8) (drill 0.4) (layers F.Cu B.Cu) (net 4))
 (segment (start 137.5 105.5) (end 142.5 105.5) (width 0.25) (layer B.Cu) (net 4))
 (segment (start 142.5 105.5) (end 142.987347 105.987347) (width 0.25) (layer B.Cu) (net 4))
 (segment (start 137 105) (end 137.5 105.5) (width 0.25) (layer F.Cu) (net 4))
 (segment (start 135 105) (end 137 105) (width 0.25) (layer F.Cu) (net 4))
 (segment (start 134.37 113.45) (end 133.96 113.04) (width 0.25) (layer B.Cu) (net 5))
 (segment (start 140.5 113.45) (end 134.37 113.45) (width 0.25) (layer B.Cu) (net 5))
 (via (at 140.5 109.5) (size 0.8) (drill 0.4) (layers F.Cu B.Cu) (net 5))
 (segment (start 146.42 97) (end 146.42 103.58) (width 0.25) (layer B.Cu) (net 5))
 (segment (start 146.42 103.58) (end 140.5 109.5) (width 0.25) (layer B.Cu) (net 5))
 (via (at 140.5 113.45) (size 0.8) (drill 0.4) (layers F.Cu B.Cu) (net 5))
 (segment (start 140.5 109.5) (end 140.5 113.45) (width 0.25) (layer F.Cu) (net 5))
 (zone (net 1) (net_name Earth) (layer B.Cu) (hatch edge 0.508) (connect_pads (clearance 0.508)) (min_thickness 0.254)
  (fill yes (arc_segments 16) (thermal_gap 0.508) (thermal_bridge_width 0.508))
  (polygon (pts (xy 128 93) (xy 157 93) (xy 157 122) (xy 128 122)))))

